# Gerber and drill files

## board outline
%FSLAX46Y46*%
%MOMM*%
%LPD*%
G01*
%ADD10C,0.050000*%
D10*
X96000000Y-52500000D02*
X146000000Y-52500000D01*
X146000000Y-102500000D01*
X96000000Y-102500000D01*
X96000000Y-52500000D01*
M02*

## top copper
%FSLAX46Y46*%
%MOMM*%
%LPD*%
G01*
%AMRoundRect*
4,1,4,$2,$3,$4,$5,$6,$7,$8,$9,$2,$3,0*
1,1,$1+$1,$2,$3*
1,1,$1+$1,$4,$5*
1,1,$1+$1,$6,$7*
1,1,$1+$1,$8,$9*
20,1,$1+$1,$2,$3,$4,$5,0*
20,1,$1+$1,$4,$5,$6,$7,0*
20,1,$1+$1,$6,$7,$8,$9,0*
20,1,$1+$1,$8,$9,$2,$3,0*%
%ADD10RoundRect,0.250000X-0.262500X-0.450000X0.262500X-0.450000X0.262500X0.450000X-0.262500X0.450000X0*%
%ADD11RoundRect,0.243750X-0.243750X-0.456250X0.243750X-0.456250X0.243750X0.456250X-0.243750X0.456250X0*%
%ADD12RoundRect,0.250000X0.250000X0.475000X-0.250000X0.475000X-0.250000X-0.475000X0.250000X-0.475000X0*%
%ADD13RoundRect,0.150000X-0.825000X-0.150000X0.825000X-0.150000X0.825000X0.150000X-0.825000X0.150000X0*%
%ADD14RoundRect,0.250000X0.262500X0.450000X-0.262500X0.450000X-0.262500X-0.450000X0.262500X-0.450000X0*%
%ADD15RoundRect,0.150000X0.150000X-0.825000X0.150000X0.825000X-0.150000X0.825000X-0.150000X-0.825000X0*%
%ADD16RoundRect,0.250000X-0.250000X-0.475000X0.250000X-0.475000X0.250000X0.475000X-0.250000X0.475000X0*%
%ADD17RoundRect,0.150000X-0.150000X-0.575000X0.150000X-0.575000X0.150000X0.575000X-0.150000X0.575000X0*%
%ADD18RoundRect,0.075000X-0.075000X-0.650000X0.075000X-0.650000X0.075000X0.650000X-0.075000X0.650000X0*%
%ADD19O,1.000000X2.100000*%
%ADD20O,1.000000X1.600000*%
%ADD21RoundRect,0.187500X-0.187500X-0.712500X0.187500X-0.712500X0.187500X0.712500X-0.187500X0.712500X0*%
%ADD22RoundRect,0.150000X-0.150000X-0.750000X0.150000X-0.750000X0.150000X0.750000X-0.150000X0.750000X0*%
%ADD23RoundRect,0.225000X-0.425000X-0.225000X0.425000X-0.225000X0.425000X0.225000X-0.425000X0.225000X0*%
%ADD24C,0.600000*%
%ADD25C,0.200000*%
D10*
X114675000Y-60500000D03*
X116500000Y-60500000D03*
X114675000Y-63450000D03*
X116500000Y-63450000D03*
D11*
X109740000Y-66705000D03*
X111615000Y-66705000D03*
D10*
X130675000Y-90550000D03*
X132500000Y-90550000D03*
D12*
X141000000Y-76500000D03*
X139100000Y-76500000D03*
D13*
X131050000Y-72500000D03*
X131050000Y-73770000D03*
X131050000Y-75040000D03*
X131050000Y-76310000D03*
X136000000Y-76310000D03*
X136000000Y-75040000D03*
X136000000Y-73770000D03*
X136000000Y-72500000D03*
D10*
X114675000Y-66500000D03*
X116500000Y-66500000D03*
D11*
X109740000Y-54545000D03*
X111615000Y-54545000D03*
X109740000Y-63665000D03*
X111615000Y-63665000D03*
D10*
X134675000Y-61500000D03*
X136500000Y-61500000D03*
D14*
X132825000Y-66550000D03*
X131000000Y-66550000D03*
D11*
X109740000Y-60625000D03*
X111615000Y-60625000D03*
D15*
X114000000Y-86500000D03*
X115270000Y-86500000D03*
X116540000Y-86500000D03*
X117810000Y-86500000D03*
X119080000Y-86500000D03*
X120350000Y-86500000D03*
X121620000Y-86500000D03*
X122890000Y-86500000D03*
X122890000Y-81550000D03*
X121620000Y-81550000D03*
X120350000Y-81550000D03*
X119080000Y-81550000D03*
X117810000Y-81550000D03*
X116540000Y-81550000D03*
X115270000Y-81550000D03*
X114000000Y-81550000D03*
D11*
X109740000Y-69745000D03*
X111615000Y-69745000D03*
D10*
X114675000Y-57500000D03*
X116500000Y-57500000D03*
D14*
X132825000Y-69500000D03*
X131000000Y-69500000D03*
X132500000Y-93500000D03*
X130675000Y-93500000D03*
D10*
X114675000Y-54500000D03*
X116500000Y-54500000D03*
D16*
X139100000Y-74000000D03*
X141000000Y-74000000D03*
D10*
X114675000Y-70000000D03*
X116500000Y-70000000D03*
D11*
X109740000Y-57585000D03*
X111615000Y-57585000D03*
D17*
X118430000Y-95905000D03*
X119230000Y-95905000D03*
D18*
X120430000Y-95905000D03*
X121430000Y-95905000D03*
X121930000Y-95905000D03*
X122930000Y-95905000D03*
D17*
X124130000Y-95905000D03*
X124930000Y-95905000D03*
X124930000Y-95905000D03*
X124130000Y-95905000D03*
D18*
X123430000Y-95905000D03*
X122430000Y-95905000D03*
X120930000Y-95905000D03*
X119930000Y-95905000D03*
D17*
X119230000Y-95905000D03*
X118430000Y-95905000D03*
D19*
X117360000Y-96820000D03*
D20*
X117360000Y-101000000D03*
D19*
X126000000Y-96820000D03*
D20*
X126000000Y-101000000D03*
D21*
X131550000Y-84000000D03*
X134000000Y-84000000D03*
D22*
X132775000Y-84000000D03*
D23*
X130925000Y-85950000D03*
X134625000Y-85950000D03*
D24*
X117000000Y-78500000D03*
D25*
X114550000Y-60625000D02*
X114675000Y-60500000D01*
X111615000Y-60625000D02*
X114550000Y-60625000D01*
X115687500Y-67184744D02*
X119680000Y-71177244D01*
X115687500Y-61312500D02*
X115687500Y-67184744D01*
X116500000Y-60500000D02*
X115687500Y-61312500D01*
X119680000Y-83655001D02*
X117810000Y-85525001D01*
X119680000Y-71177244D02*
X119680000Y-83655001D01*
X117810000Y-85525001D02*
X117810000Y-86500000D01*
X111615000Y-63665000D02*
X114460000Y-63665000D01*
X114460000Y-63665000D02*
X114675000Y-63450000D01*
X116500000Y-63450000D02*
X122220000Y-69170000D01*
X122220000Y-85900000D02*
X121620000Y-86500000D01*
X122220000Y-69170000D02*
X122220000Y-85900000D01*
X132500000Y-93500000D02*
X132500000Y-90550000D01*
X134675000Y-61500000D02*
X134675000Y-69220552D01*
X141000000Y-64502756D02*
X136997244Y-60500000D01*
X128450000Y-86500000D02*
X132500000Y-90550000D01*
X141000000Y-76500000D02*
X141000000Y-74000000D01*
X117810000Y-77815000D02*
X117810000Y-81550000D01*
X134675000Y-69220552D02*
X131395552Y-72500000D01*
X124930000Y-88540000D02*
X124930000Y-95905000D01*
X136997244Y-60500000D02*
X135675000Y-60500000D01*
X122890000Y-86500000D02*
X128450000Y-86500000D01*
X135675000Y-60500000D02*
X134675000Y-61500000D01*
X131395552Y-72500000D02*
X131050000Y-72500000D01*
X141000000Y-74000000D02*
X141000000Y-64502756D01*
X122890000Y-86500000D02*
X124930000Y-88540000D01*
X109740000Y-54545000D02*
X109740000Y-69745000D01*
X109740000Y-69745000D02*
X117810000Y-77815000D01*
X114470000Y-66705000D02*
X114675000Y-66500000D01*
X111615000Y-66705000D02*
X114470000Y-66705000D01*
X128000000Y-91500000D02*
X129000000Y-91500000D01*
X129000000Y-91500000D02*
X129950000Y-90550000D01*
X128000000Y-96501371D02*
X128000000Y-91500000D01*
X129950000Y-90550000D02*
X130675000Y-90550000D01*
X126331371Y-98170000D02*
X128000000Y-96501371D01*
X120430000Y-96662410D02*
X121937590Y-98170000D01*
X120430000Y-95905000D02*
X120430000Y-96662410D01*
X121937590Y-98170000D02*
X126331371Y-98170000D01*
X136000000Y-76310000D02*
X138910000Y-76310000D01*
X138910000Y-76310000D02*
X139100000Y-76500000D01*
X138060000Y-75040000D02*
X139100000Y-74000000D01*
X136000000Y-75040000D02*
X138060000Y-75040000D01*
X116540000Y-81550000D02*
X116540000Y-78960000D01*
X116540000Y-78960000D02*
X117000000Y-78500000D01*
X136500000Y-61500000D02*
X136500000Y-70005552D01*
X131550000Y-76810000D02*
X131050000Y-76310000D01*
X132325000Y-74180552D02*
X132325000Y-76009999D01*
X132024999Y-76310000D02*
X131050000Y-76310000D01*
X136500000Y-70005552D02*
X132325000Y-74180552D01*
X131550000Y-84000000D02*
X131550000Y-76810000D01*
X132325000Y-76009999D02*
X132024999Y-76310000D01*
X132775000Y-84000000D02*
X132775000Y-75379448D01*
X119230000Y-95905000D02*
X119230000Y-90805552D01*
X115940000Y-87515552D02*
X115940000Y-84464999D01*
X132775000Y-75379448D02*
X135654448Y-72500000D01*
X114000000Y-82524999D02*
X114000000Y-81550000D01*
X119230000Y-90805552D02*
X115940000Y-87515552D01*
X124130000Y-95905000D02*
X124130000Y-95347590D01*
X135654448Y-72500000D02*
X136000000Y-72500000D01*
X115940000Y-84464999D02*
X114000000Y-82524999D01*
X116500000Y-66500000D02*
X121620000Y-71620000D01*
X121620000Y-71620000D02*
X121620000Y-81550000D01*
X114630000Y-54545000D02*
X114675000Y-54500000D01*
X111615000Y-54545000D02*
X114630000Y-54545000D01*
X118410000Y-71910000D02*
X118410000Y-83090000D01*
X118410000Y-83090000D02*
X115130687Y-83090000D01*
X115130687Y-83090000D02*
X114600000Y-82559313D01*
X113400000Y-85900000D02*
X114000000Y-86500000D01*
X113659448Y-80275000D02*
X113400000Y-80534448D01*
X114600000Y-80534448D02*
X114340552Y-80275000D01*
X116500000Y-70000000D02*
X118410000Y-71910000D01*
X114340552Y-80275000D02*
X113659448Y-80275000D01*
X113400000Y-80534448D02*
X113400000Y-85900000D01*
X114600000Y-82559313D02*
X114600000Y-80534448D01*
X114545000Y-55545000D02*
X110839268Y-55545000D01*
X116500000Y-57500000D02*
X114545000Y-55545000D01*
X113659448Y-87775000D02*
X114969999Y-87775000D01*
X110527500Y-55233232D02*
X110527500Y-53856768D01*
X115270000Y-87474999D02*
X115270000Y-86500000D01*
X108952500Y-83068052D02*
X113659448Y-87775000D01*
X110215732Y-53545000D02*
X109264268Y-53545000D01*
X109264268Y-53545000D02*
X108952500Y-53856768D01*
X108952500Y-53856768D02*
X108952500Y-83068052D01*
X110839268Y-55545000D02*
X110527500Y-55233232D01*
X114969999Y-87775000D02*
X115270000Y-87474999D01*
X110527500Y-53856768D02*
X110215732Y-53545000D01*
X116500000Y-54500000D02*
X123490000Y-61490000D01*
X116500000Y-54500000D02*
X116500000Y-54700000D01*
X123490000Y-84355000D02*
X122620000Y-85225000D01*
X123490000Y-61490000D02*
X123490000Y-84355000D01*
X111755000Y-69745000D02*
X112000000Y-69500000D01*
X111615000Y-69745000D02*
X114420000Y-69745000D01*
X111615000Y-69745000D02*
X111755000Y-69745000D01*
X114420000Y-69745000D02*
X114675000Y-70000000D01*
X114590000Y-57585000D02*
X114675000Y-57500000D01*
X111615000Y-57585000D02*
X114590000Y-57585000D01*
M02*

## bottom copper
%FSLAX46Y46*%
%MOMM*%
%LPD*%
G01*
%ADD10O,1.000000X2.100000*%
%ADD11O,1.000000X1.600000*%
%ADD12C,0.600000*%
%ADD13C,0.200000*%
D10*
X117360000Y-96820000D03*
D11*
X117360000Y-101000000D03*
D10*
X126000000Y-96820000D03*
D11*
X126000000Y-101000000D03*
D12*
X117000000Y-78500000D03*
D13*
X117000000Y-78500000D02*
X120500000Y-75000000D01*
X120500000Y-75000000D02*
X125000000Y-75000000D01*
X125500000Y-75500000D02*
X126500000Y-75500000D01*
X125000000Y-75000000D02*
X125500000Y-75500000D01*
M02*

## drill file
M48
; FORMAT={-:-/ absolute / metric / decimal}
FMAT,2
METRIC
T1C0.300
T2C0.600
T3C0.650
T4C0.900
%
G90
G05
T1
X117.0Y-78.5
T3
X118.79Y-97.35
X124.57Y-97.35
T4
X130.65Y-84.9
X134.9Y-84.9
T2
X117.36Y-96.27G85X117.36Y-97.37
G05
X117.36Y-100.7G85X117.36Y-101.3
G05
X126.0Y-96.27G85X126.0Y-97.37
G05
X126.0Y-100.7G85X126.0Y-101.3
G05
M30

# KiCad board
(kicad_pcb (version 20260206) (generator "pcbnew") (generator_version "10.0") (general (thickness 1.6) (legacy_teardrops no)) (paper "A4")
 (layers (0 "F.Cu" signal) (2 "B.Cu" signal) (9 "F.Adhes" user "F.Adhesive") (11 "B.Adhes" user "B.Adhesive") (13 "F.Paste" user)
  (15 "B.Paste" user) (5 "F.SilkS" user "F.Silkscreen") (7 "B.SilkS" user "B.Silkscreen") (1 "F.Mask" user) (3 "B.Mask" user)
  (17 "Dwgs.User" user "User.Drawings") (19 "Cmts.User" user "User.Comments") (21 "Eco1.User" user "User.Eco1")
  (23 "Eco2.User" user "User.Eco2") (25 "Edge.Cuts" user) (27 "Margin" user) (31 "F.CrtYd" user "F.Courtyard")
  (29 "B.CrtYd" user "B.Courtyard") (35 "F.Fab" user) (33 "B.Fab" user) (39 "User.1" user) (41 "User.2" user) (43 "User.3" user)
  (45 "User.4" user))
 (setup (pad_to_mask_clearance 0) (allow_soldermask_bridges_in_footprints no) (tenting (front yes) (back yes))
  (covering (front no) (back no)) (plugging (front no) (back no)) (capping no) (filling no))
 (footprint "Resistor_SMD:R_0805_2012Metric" (layer "F.Cu") (at 115.5875 60.5)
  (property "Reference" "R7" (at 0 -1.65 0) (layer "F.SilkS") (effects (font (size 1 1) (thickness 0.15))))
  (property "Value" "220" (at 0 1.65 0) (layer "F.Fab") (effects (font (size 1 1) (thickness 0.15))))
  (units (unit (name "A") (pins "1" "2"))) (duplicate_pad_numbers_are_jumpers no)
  (pad "1" smd roundrect (at -0.9125 0) (size 1.025 1.4) (layers "F.Cu" "F.Mask" "F.Paste") (roundrect_rratio 0.243902) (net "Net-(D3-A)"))
  (pad "2" smd roundrect (at 0.9125 0) (size 1.025 1.4) (layers "F.Cu" "F.Mask" "F.Paste") (roundrect_rratio 0.243902) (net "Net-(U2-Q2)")))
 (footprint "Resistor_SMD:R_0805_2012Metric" (layer "F.Cu") (at 115.5875 63.45)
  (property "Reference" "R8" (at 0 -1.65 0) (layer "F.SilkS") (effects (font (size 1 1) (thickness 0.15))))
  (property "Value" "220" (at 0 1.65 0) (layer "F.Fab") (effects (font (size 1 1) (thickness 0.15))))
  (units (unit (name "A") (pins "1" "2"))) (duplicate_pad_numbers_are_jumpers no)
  (pad "1" smd roundrect (at -0.9125 0) (size 1.025 1.4) (layers "F.Cu" "F.Mask" "F.Paste") (roundrect_rratio 0.243902) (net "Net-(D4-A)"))
  (pad "2" smd roundrect (at 0.9125 0) (size 1.025 1.4) (layers "F.Cu" "F.Mask" "F.Paste") (roundrect_rratio 0.243902) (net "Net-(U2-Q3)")))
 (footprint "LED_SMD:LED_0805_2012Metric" (layer "F.Cu") (at 110.6775 66.705)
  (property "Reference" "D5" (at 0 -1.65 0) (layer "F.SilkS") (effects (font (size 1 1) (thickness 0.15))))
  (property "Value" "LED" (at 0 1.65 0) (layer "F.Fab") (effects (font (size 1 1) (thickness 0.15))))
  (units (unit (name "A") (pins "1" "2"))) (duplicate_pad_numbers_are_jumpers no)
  (pad "1" smd roundrect (at -0.9375 0) (size 0.975 1.4) (layers "F.Cu" "F.Mask" "F.Paste") (roundrect_rratio 0.25) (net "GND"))
  (pad "2" smd roundrect (at 0.9375 0) (size 0.975 1.4) (layers "F.Cu" "F.Mask" "F.Paste") (roundrect_rratio 0.25) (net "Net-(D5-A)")))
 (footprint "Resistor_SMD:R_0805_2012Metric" (layer "F.Cu") (at 131.5875 90.55)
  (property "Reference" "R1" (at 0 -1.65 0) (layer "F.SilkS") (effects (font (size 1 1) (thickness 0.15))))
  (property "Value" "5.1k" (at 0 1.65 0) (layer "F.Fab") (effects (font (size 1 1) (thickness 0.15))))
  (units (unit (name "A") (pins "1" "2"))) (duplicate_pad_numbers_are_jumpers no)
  (pad "1" smd roundrect (at -0.9125 0) (size 1.025 1.4) (layers "F.Cu" "F.Mask" "F.Paste") (roundrect_rratio 0.243902) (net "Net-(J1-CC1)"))
  (pad "2" smd roundrect (at 0.9125 0) (size 1.025 1.4) (layers "F.Cu" "F.Mask" "F.Paste") (roundrect_rratio 0.243902) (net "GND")))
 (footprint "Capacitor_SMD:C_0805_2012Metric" (layer "F.Cu") (at 140.05 76.5 180)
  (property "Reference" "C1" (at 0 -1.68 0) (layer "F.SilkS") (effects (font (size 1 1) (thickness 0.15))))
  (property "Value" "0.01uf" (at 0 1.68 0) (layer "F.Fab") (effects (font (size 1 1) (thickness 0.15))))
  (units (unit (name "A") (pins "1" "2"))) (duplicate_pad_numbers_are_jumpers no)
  (pad "1" smd roundrect (at -0.95 0 180) (size 1 1.45) (layers "F.Cu" "F.Mask" "F.Paste") (roundrect_rratio 0.25) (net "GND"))
  (pad "2" smd roundrect (at 0.95 0 180) (size 1 1.45) (layers "F.Cu" "F.Mask" "F.Paste") (roundrect_rratio 0.25) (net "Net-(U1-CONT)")))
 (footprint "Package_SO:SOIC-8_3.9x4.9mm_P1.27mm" (layer "F.Cu") (at 133.525 74.405)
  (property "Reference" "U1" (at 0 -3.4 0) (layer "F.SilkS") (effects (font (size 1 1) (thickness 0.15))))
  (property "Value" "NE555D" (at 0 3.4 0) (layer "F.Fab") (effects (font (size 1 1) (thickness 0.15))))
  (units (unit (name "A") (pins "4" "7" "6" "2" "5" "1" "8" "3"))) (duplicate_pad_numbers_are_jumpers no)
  (pad "1" smd roundrect (at -2.475 -1.905) (size 1.95 0.6) (layers "F.Cu" "F.Mask" "F.Paste") (roundrect_rratio 0.25) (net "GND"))
  (pad "2" smd roundrect (at -2.475 -0.635) (size 1.95 0.6) (layers "F.Cu" "F.Mask" "F.Paste") (roundrect_rratio 0.25)
   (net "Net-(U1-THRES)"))
  (pad "3" smd roundrect (at -2.475 0.635) (size 1.95 0.6) (layers "F.Cu" "F.Mask" "F.Paste") (roundrect_rratio 0.25) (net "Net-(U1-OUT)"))
  (pad "4" smd roundrect (at -2.475 1.905) (size 1.95 0.6) (layers "F.Cu" "F.Mask" "F.Paste") (roundrect_rratio 0.25)
   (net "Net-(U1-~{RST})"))
  (pad "5" smd roundrect (at 2.475 1.905) (size 1.95 0.6) (layers "F.Cu" "F.Mask" "F.Paste") (roundrect_rratio 0.25) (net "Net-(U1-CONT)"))
  (pad "6" smd roundrect (at 2.475 0.635) (size 1.95 0.6) (layers "F.Cu" "F.Mask" "F.Paste") (roundrect_rratio 0.25) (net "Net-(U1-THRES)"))
  (pad "7" smd roundrect (at 2.475 -0.635) (size 1.95 0.6) (layers "F.Cu" "F.Mask" "F.Paste") (roundrect_rratio 0.25) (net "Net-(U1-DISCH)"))
  (pad "8" smd roundrect (at 2.475 -1.905) (size 1.95 0.6) (layers "F.Cu" "F.Mask" "F.Paste") (roundrect_rratio 0.25) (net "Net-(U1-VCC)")))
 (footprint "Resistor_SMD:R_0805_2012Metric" (layer "F.Cu") (at 115.5875 66.5)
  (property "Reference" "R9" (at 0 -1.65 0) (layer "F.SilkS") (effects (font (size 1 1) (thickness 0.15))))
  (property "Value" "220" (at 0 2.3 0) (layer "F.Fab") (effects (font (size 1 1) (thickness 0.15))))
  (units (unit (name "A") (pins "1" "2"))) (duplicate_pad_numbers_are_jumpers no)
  (pad "1" smd roundrect (at -0.9125 0) (size 1.025 1.4) (layers "F.Cu" "F.Mask" "F.Paste") (roundrect_rratio 0.243902) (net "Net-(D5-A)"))
  (pad "2" smd roundrect (at 0.9125 0) (size 1.025 1.4) (layers "F.Cu" "F.Mask" "F.Paste") (roundrect_rratio 0.243902) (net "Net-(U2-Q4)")))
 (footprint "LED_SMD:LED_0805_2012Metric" (layer "F.Cu") (at 110.6775 54.545)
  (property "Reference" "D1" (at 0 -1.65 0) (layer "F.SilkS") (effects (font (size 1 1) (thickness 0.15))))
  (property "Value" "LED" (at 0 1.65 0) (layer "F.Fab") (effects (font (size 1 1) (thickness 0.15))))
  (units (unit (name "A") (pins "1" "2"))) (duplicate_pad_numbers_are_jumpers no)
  (pad "1" smd roundrect (at -0.9375 0) (size 0.975 1.4) (layers "F.Cu" "F.Mask" "F.Paste") (roundrect_rratio 0.25) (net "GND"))
  (pad "2" smd roundrect (at 0.9375 0) (size 0.975 1.4) (layers "F.Cu" "F.Mask" "F.Paste") (roundrect_rratio 0.25) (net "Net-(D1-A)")))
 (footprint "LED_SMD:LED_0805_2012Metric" (layer "F.Cu") (at 110.6775 63.665)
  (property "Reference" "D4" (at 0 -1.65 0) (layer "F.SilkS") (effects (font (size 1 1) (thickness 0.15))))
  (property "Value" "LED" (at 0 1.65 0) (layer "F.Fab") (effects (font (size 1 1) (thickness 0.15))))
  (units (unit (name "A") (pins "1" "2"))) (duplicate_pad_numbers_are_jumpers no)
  (pad "1" smd roundrect (at -0.9375 0) (size 0.975 1.4) (layers "F.Cu" "F.Mask" "F.Paste") (roundrect_rratio 0.25) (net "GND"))
  (pad "2" smd roundrect (at 0.9375 0) (size 0.975 1.4) (layers "F.Cu" "F.Mask" "F.Paste") (roundrect_rratio 0.25) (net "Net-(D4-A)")))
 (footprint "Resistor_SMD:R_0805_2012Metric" (layer "F.Cu") (at 135.5875 61.5)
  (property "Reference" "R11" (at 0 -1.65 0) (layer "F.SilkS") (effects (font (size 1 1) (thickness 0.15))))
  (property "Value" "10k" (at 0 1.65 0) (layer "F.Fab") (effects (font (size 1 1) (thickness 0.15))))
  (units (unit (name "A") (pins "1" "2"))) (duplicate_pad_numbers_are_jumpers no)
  (pad "1" smd roundrect (at -0.9125 0) (size 1.025 1.4) (layers "F.Cu" "F.Mask" "F.Paste") (roundrect_rratio 0.243902) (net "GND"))
  (pad "2" smd roundrect (at 0.9125 0) (size 1.025 1.4) (layers "F.Cu" "F.Mask" "F.Paste") (roundrect_rratio 0.243902)
   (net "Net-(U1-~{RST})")))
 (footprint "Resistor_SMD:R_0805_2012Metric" (layer "F.Cu") (at 131.9125 66.55 180)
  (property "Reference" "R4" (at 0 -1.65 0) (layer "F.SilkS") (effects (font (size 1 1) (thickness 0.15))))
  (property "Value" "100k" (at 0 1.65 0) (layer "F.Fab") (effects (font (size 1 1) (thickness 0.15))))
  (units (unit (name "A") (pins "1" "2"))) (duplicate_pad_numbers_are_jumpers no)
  (pad "1" smd roundrect (at -0.9125 0 180) (size 1.025 1.4) (layers "F.Cu" "F.Mask" "F.Paste") (roundrect_rratio 0.243902)
   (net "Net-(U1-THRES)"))
  (pad "2" smd roundrect (at 0.9125 0 180) (size 1.025 1.4) (layers "F.Cu" "F.Mask" "F.Paste") (roundrect_rratio 0.243902)
   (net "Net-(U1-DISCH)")))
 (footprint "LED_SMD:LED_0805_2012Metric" (layer "F.Cu") (at 110.6775 60.625)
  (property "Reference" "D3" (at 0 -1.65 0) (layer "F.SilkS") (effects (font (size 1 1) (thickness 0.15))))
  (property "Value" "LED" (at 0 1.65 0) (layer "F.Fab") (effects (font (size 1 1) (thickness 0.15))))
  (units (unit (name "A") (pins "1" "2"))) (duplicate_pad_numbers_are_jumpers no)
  (pad "1" smd roundrect (at -0.9375 0) (size 0.975 1.4) (layers "F.Cu" "F.Mask" "F.Paste") (roundrect_rratio 0.25) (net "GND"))
  (pad "2" smd roundrect (at 0.9375 0) (size 0.975 1.4) (layers "F.Cu" "F.Mask" "F.Paste") (roundrect_rratio 0.25) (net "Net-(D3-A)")))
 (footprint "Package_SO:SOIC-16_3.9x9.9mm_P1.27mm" (layer "F.Cu") (at 118.445 84.025 90)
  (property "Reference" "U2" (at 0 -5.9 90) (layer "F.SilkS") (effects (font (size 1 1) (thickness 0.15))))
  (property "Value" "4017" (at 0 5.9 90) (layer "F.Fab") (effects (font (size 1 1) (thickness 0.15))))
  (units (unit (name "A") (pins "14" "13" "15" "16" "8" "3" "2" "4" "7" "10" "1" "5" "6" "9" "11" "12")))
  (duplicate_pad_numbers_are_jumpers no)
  (pad "1" smd roundrect (at -2.475 -4.445 90) (size 1.95 0.6) (layers "F.Cu" "F.Mask" "F.Paste") (roundrect_rratio 0.25)
   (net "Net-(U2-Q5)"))
  (pad "2" smd roundrect (at -2.475 -3.175 90) (size 1.95 0.6) (layers "F.Cu" "F.Mask" "F.Paste") (roundrect_rratio 0.25)
   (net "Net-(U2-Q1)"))
  (pad "3" smd roundrect (at -2.475 -1.905 90) (size 1.95 0.6) (layers "F.Cu" "F.Mask" "F.Paste") (roundrect_rratio 0.25)
   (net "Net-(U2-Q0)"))
  (pad "4" smd roundrect (at -2.475 -0.635 90) (size 1.95 0.6) (layers "F.Cu" "F.Mask" "F.Paste") (roundrect_rratio 0.25)
   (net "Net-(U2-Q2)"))
  (pad "5" smd roundrect (at -2.475 0.635 90) (size 1.95 0.6) (layers "F.Cu" "F.Mask" "F.Paste") (roundrect_rratio 0.25) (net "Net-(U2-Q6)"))
  (pad "6" smd roundrect (at -2.475 1.905 90) (size 1.95 0.6) (layers "F.Cu" "F.Mask" "F.Paste") (roundrect_rratio 0.25)
   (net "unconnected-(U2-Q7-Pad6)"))
  (pad "7" smd roundrect (at -2.475 3.175 90) (size 1.95 0.6) (layers "F.Cu" "F.Mask" "F.Paste") (roundrect_rratio 0.25) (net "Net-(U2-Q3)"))
  (pad "8" smd roundrect (at -2.475 4.445 90) (size 1.95 0.6) (layers "F.Cu" "F.Mask" "F.Paste") (roundrect_rratio 0.25) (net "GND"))
  (pad "9" smd roundrect (at 2.475 4.445 90) (size 1.95 0.6) (layers "F.Cu" "F.Mask" "F.Paste") (roundrect_rratio 0.25)
   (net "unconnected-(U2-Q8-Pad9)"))
  (pad "10" smd roundrect (at 2.475 3.175 90) (size 1.95 0.6) (layers "F.Cu" "F.Mask" "F.Paste") (roundrect_rratio 0.25) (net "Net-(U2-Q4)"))
  (pad "11" smd roundrect (at 2.475 1.905 90) (size 1.95 0.6) (layers "F.Cu" "F.Mask" "F.Paste") (roundrect_rratio 0.25)
   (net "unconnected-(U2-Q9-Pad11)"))
  (pad "12" smd roundrect (at 2.475 0.635 90) (size 1.95 0.6) (layers "F.Cu" "F.Mask" "F.Paste") (roundrect_rratio 0.25)
   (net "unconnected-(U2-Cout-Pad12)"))
  (pad "13" smd roundrect (at 2.475 -0.635 90) (size 1.95 0.6) (layers "F.Cu" "F.Mask" "F.Paste") (roundrect_rratio 0.25) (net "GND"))
  (pad "14" smd roundrect (at 2.475 -1.905 90) (size 1.95 0.6) (layers "F.Cu" "F.Mask" "F.Paste") (roundrect_rratio 0.25)
   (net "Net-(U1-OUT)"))
  (pad "15" smd roundrect (at 2.475 -3.175 90) (size 1.95 0.6) (layers "F.Cu" "F.Mask" "F.Paste") (roundrect_rratio 0.25)
   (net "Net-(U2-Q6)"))
  (pad "16" smd roundrect (at 2.475 -4.445 90) (size 1.95 0.6) (layers "F.Cu" "F.Mask" "F.Paste") (roundrect_rratio 0.25)
   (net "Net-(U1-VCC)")))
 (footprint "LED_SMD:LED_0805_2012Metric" (layer "F.Cu") (at 110.6775 69.745)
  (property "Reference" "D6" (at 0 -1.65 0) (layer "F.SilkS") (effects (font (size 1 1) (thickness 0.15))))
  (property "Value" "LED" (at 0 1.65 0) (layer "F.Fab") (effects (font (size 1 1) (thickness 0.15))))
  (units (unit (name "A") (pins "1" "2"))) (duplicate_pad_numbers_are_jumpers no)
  (pad "1" smd roundrect (at -0.9375 0) (size 0.975 1.4) (layers "F.Cu" "F.Mask" "F.Paste") (roundrect_rratio 0.25) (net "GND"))
  (pad "2" smd roundrect (at 0.9375 0) (size 0.975 1.4) (layers "F.Cu" "F.Mask" "F.Paste") (roundrect_rratio 0.25) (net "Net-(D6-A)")))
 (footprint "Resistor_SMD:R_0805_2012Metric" (layer "F.Cu") (at 115.5875 57.5)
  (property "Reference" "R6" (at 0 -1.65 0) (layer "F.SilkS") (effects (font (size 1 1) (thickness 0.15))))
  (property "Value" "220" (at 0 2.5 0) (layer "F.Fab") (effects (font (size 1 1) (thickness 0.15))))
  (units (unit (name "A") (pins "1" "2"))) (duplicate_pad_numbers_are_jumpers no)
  (pad "1" smd roundrect (at -0.9125 0) (size 1.025 1.4) (layers "F.Cu" "F.Mask" "F.Paste") (roundrect_rratio 0.243902) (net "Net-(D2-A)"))
  (pad "2" smd roundrect (at 0.9125 0) (size 1.025 1.4) (layers "F.Cu" "F.Mask" "F.Paste") (roundrect_rratio 0.243902) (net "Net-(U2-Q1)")))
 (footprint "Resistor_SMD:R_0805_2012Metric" (layer "F.Cu") (at 131.9125 69.5 180)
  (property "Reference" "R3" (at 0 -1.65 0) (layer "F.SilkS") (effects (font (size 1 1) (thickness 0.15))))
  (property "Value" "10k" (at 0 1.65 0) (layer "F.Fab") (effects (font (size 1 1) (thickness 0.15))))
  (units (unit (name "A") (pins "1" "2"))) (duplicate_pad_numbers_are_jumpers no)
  (pad "1" smd roundrect (at -0.9125 0 180) (size 1.025 1.4) (layers "F.Cu" "F.Mask" "F.Paste") (roundrect_rratio 0.243902)
   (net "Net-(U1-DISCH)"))
  (pad "2" smd roundrect (at 0.9125 0 180) (size 1.025 1.4) (layers "F.Cu" "F.Mask" "F.Paste") (roundrect_rratio 0.243902)
   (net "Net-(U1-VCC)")))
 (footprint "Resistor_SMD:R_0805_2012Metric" (layer "F.Cu") (at 131.5875 93.5 180)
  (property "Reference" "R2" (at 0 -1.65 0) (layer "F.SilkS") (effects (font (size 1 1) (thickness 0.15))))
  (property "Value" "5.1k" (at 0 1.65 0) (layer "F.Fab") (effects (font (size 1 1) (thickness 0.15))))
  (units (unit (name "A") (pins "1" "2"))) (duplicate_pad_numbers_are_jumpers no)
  (pad "1" smd roundrect (at -0.9125 0 180) (size 1.025 1.4) (layers "F.Cu" "F.Mask" "F.Paste") (roundrect_rratio 0.243902) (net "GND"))
  (pad "2" smd roundrect (at 0.9125 0 180) (size 1.025 1.4) (layers "F.Cu" "F.Mask" "F.Paste") (roundrect_rratio 0.243902)
   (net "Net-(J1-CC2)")))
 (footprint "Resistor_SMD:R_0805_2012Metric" (layer "F.Cu") (at 115.5875 54.5)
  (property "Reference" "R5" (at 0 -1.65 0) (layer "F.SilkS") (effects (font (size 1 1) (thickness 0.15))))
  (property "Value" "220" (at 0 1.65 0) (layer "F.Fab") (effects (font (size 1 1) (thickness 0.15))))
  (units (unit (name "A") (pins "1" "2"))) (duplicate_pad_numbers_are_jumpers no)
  (pad "1" smd roundrect (at -0.9125 0) (size 1.025 1.4) (layers "F.Cu" "F.Mask" "F.Paste") (roundrect_rratio 0.243902) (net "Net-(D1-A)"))
  (pad "2" smd roundrect (at 0.9125 0) (size 1.025 1.4) (layers "F.Cu" "F.Mask" "F.Paste") (roundrect_rratio 0.243902) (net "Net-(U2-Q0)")))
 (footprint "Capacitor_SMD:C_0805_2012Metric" (layer "F.Cu") (at 140.05 74)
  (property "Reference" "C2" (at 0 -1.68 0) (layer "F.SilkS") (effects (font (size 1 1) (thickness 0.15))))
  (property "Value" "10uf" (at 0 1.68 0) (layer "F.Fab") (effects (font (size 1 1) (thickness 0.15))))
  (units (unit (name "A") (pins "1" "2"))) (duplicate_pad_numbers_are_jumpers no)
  (pad "1" smd roundrect (at -0.95 0) (size 1 1.45) (layers "F.Cu" "F.Mask" "F.Paste") (roundrect_rratio 0.25) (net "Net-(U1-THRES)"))
  (pad "2" smd roundrect (at 0.95 0) (size 1 1.45) (layers "F.Cu" "F.Mask" "F.Paste") (roundrect_rratio 0.25) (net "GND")))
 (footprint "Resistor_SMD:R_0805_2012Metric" (layer "F.Cu") (at 115.5875 70)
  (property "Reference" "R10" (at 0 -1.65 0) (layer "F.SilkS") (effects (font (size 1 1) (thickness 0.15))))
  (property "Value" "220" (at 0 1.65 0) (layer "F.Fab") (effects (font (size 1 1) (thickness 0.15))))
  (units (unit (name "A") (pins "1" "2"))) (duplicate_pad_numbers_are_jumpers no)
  (pad "1" smd roundrect (at -0.9125 0) (size 1.025 1.4) (layers "F.Cu" "F.Mask" "F.Paste") (roundrect_rratio 0.243902) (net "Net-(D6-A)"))
  (pad "2" smd roundrect (at 0.9125 0) (size 1.025 1.4) (layers "F.Cu" "F.Mask" "F.Paste") (roundrect_rratio 0.243902) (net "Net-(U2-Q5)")))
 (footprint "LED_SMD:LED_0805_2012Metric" (layer "F.Cu") (at 110.6775 57.585)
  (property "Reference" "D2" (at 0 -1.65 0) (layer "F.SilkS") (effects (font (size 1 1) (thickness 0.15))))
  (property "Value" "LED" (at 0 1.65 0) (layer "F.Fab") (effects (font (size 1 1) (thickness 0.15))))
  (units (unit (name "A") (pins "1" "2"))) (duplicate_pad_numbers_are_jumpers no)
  (pad "1" smd roundrect (at -0.9375 0) (size 0.975 1.4) (layers "F.Cu" "F.Mask" "F.Paste") (roundrect_rratio 0.25) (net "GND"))
  (pad "2" smd roundrect (at 0.9375 0) (size 0.975 1.4) (layers "F.Cu" "F.Mask" "F.Paste") (roundrect_rratio 0.25) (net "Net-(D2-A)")))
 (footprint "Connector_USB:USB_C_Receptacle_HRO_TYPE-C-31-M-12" (layer "F.Cu") (at 121.68 99.95)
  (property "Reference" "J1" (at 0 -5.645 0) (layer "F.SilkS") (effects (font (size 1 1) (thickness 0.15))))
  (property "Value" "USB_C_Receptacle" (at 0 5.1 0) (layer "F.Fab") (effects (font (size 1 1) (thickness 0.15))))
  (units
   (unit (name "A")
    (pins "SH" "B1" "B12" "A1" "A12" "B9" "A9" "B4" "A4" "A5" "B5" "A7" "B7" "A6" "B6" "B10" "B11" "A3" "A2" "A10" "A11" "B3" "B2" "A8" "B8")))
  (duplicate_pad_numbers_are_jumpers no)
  (pad "" np_thru_hole circle (at -2.89 -2.6) (size 0.65 0.65) (drill 0.65) (layers "*.Cu" "*.Mask"))
  (pad "" np_thru_hole circle (at 2.89 -2.6) (size 0.65 0.65) (drill 0.65) (layers "*.Cu" "*.Mask"))
  (pad "A1" smd roundrect (at -3.25 -4.045) (size 0.6 1.45) (layers "F.Cu" "F.Mask" "F.Paste") (roundrect_rratio 0.25) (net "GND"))
  (pad "A4" smd roundrect (at -2.45 -4.045) (size 0.6 1.45) (layers "F.Cu" "F.Mask" "F.Paste") (roundrect_rratio 0.25) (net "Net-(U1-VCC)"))
  (pad "A5" smd roundrect (at -1.25 -4.045) (size 0.3 1.45) (layers "F.Cu" "F.Mask" "F.Paste") (roundrect_rratio 0.25) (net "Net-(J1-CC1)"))
  (pad "A6" smd roundrect (at -0.25 -4.045) (size 0.3 1.45) (layers "F.Cu" "F.Mask" "F.Paste") (roundrect_rratio 0.25)
   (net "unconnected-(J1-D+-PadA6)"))
  (pad "A7" smd roundrect (at 0.25 -4.045) (size 0.3 1.45) (layers "F.Cu" "F.Mask" "F.Paste") (roundrect_rratio 0.25)
   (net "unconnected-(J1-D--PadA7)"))
  (pad "A8" smd roundrect (at 1.25 -4.045) (size 0.3 1.45) (layers "F.Cu" "F.Mask" "F.Paste") (roundrect_rratio 0.25)
   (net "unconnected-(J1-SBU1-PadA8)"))
  (pad "A9" smd roundrect (at 2.45 -4.045) (size 0.6 1.45) (layers "F.Cu" "F.Mask" "F.Paste") (roundrect_rratio 0.25) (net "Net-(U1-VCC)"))
  (pad "A12" smd roundrect (at 3.25 -4.045) (size 0.6 1.45) (layers "F.Cu" "F.Mask" "F.Paste") (roundrect_rratio 0.25) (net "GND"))
  (pad "B1" smd roundrect (at 3.25 -4.045) (size 0.6 1.45) (layers "F.Cu" "F.Mask" "F.Paste") (roundrect_rratio 0.25) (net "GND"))
  (pad "B4" smd roundrect (at 2.45 -4.045) (size 0.6 1.45) (layers "F.Cu" "F.Mask" "F.Paste") (roundrect_rratio 0.25) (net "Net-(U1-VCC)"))
  (pad "B5" smd roundrect (at 1.75 -4.045) (size 0.3 1.45) (layers "F.Cu" "F.Mask" "F.Paste") (roundrect_rratio 0.25) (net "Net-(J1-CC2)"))
  (pad "B6" smd roundrect (at 0.75 -4.045) (size 0.3 1.45) (layers "F.Cu" "F.Mask" "F.Paste") (roundrect_rratio 0.25)
   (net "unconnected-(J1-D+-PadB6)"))
  (pad "B7" smd roundrect (at -0.75 -4.045) (size 0.3 1.45) (layers "F.Cu" "F.Mask" "F.Paste") (roundrect_rratio 0.25)
   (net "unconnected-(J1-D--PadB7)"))
  (pad "B8" smd roundrect (at -1.75 -4.045) (size 0.3 1.45) (layers "F.Cu" "F.Mask" "F.Paste") (roundrect_rratio 0.25)
   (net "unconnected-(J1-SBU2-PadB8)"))
  (pad "B9" smd roundrect (at -2.45 -4.045) (size 0.6 1.45) (layers "F.Cu" "F.Mask" "F.Paste") (roundrect_rratio 0.25) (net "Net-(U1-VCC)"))
  (pad "B12" smd roundrect (at -3.25 -4.045) (size 0.6 1.45) (layers "F.Cu" "F.Mask" "F.Paste") (roundrect_rratio 0.25) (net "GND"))
  (pad "SH" thru_hole oval (at -4.32 -3.13) (size 1 2.1) (drill oval 0.6 1.7) (layers "*.Cu" "*.Mask") (remove_unused_layers no)
   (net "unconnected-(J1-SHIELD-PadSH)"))
  (pad "SH" thru_hole oval (at -4.32 1.05) (size 1 1.6) (drill oval 0.6 1.2) (layers "*.Cu" "*.Mask") (remove_unused_layers no)
   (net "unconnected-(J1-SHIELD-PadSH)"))
  (pad "SH" thru_hole oval (at 4.32 -3.13) (size 1 2.1) (drill oval 0.6 1.7) (layers "*.Cu" "*.Mask") (remove_unused_layers no)
   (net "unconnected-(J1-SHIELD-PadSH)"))
  (pad "SH" thru_hole oval (at 4.32 1.05) (size 1 1.6) (drill oval 0.6 1.2) (layers "*.Cu" "*.Mask") (remove_unused_layers no)
   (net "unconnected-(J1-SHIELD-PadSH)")))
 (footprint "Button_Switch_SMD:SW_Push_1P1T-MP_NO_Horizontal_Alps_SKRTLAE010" (layer "F.Cu") (at 132.775 84.9)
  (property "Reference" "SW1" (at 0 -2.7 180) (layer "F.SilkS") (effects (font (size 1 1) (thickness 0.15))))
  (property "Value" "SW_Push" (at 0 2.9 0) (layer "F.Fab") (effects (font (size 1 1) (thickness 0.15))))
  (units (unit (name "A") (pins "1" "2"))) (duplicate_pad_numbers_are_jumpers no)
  (pad "" np_thru_hole circle (at -2.125 0) (size 0.9 0.9) (drill 0.9) (layers "*.Cu" "*.Mask"))
  (pad "" np_thru_hole circle (at 2.125 0) (size 0.9 0.9) (drill 0.9) (layers "*.Cu" "*.Mask"))
  (pad "1" smd roundrect (at -1.225 -0.9) (size 0.75 1.8) (layers "F.Cu" "F.Mask" "F.Paste") (roundrect_rratio 0.25) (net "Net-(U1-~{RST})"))
  (pad "1" smd roundrect (at 1.225 -0.9) (size 0.75 1.8) (layers "F.Cu" "F.Mask" "F.Paste") (roundrect_rratio 0.25) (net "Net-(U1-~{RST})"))
  (pad "2" smd roundrect (at 0 -0.9) (size 0.6 1.8) (layers "F.Cu" "F.Mask" "F.Paste") (roundrect_rratio 0.25) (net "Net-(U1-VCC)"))
  (pad "MP" smd roundrect (at -1.85 1.05) (size 1.3 0.9) (layers "F.Cu" "F.Mask" "F.Paste") (roundrect_rratio 0.25))
  (pad "MP" smd roundrect (at 1.85 1.05) (size 1.3 0.9) (layers "F.Cu" "F.Mask" "F.Paste") (roundrect_rratio 0.25)))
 (gr_rect (start 96 52.5) (end 146 102.5) (stroke (width 0.05) (type solid)) (fill no) (layer "Edge.Cuts"))
 (segment (start 114.55 60.625) (end 114.675 60.5) (width 0.2) (layer "F.Cu") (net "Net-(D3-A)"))
 (segment (start 111.615 60.625) (end 114.55 60.625) (width 0.2) (layer "F.Cu") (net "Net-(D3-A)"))
 (segment (start 115.6875 67.184744) (end 119.68 71.177244) (width 0.2) (layer "F.Cu") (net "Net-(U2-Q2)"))
 (segment (start 115.6875 61.3125) (end 115.6875 67.184744) (width 0.2) (layer "F.Cu") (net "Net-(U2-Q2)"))
 (segment (start 116.5 60.5) (end 115.6875 61.3125) (width 0.2) (layer "F.Cu") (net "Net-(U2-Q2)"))
 (segment (start 119.68 83.655001) (end 117.81 85.525001) (width 0.2) (layer "F.Cu") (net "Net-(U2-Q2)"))
 (segment (start 119.68 71.177244) (end 119.68 83.655001) (width 0.2) (layer "F.Cu") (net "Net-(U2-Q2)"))
 (segment (start 117.81 85.525001) (end 117.81 86.5) (width 0.2) (layer "F.Cu") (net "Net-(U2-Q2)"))
 (segment (start 111.615 63.665) (end 114.46 63.665) (width 0.2) (layer "F.Cu") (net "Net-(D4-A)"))
 (segment (start 114.46 63.665) (end 114.675 63.45) (width 0.2) (layer "F.Cu") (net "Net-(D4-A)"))
 (segment (start 116.5 63.45) (end 122.22 69.17) (width 0.2) (layer "F.Cu") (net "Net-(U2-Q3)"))
 (segment (start 122.22 85.9) (end 121.62 86.5) (width 0.2) (layer "F.Cu") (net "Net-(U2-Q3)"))
 (segment (start 122.22 69.17) (end 122.22 85.9) (width 0.2) (layer "F.Cu") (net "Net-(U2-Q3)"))
 (segment (start 132.5 93.5) (end 132.5 90.55) (width 0.2) (layer "F.Cu") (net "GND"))
 (segment (start 134.675 61.5) (end 134.675 69.220552) (width 0.2) (layer "F.Cu") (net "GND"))
 (segment (start 141 64.502756) (end 136.997244 60.5) (width 0.2) (layer "F.Cu") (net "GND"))
 (segment (start 128.45 86.5) (end 132.5 90.55) (width 0.2) (layer "F.Cu") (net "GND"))
 (segment (start 141 76.5) (end 141 74) (width 0.2) (layer "F.Cu") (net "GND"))
 (segment (start 117.81 77.815) (end 117.81 81.55) (width 0.2) (layer "F.Cu") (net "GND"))
 (segment (start 134.675 69.220552) (end 131.395552 72.5) (width 0.2) (layer "F.Cu") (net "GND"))
 (segment (start 124.93 88.54) (end 124.93 95.905) (width 0.2) (layer "F.Cu") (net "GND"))
 (segment (start 136.997244 60.5) (end 135.675 60.5) (width 0.2) (layer "F.Cu") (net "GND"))
 (segment (start 122.89 86.5) (end 128.45 86.5) (width 0.2) (layer "F.Cu") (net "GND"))
 (segment (start 135.675 60.5) (end 134.675 61.5) (width 0.2) (layer "F.Cu") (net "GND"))
 (segment (start 131.395552 72.5) (end 131.05 72.5) (width 0.2) (layer "F.Cu") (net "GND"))
 (segment (start 141 74) (end 141 64.502756) (width 0.2) (layer "F.Cu") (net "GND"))
 (segment (start 122.89 86.5) (end 124.93 88.54) (width 0.2) (layer "F.Cu") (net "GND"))
 (segment (start 109.74 54.545) (end 109.74 69.745) (width 0.2) (layer "F.Cu") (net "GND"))
 (segment (start 109.74 69.745) (end 117.81 77.815) (width 0.2) (layer "F.Cu") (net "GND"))
 (segment (start 114.47 66.705) (end 114.675 66.5) (width 0.2) (layer "F.Cu") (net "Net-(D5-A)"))
 (segment (start 111.615 66.705) (end 114.47 66.705) (width 0.2) (layer "F.Cu") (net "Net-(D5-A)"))
 (segment (start 128 91.5) (end 129 91.5) (width 0.2) (layer "F.Cu") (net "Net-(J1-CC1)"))
 (segment (start 129 91.5) (end 129.95 90.55) (width 0.2) (layer "F.Cu") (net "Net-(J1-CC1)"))
 (segment (start 128 96.501371) (end 128 91.5) (width 0.2) (layer "F.Cu") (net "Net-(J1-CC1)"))
 (segment (start 129.95 90.55) (end 130.675 90.55) (width 0.2) (layer "F.Cu") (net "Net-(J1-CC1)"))
 (segment (start 126.331371 98.17) (end 128 96.501371) (width 0.2) (layer "F.Cu") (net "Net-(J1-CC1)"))
 (segment (start 120.43 96.66241) (end 121.93759 98.17) (width 0.2) (layer "F.Cu") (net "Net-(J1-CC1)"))
 (segment (start 120.43 95.905) (end 120.43 96.66241) (width 0.2) (layer "F.Cu") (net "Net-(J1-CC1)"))
 (segment (start 121.93759 98.17) (end 126.331371 98.17) (width 0.2) (layer "F.Cu") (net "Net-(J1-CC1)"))
 (segment (start 136 76.31) (end 138.91 76.31) (width 0.2) (layer "F.Cu") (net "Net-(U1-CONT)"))
 (segment (start 138.91 76.31) (end 139.1 76.5) (width 0.2) (layer "F.Cu") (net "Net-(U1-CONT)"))
 (segment (start 138.06 75.04) (end 139.1 74) (width 0.2) (layer "F.Cu") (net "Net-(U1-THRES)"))
 (segment (start 136 75.04) (end 138.06 75.04) (width 0.2) (layer "F.Cu") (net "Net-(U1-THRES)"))
 (segment (start 116.54 81.55) (end 116.54 78.96) (width 0.2) (layer "F.Cu") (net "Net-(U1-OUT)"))
 (segment (start 116.54 78.96) (end 117 78.5) (width 0.2) (layer "F.Cu") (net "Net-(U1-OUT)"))
 (via (at 117 78.5) (size 0.6) (drill 0.3) (layers "F.Cu" "B.Cu") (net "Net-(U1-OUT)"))
 (segment (start 117 78.5) (end 120.5 75) (width 0.2) (layer "B.Cu") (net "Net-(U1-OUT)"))
 (segment (start 120.5 75) (end 125 75) (width 0.2) (layer "B.Cu") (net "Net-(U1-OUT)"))
 (segment (start 125.5 75.5) (end 126.5 75.5) (width 0.2) (layer "B.Cu") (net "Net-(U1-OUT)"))
 (segment (start 125 75) (end 125.5 75.5) (width 0.2) (layer "B.Cu") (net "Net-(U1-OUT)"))
 (segment (start 136.5 61.5) (end 136.5 70.005552) (width 0.2) (layer "F.Cu") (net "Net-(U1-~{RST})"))
 (segment (start 131.55 76.81) (end 131.05 76.31) (width 0.2) (layer "F.Cu") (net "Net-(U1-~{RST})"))
 (segment (start 132.325 74.180552) (end 132.325 76.009999) (width 0.2) (layer "F.Cu") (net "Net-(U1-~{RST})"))
 (segment (start 132.024999 76.31) (end 131.05 76.31) (width 0.2) (layer "F.Cu") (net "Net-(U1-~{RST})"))
 (segment (start 136.5 70.005552) (end 132.325 74.180552) (width 0.2) (layer "F.Cu") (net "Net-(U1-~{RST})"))
 (segment (start 131.55 84) (end 131.55 76.81) (width 0.2) (layer "F.Cu") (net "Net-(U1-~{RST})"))
 (segment (start 132.325 76.009999) (end 132.024999 76.31) (width 0.2) (layer "F.Cu") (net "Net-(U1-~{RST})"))
 (segment (start 132.775 84) (end 132.775 75.379448) (width 0.2) (layer "F.Cu") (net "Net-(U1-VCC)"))
 (segment (start 119.23 95.905) (end 119.23 90.805552) (width 0.2) (layer "F.Cu") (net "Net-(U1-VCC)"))
 (segment (start 115.94 87.515552) (end 115.94 84.464999) (width 0.2) (layer "F.Cu") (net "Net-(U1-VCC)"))
 (segment (start 132.775 75.379448) (end 135.654448 72.5) (width 0.2) (layer "F.Cu") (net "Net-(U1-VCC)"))
 (segment (start 114 82.524999) (end 114 81.55) (width 0.2) (layer "F.Cu") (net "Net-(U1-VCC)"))
 (segment (start 119.23 90.805552) (end 115.94 87.515552) (width 0.2) (layer "F.Cu") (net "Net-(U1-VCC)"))
 (segment (start 124.13 95.905) (end 124.13 95.34759) (width 0.2) (layer "F.Cu") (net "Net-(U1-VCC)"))
 (segment (start 135.654448 72.5) (end 136 72.5) (width 0.2) (layer "F.Cu") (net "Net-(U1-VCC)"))
 (segment (start 115.94 84.464999) (end 114 82.524999) (width 0.2) (layer "F.Cu") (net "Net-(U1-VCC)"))
 (segment (start 116.5 66.5) (end 121.62 71.62) (width 0.2) (layer "F.Cu") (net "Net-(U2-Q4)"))
 (segment (start 121.62 71.62) (end 121.62 81.55) (width 0.2) (layer "F.Cu") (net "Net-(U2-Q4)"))
 (segment (start 114.63 54.545) (end 114.675 54.5) (width 0.2) (layer "F.Cu") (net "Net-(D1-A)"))
 (segment (start 111.615 54.545) (end 114.63 54.545) (width 0.2) (layer "F.Cu") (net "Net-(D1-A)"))
 (segment (start 118.41 71.91) (end 118.41 83.09) (width 0.2) (layer "F.Cu") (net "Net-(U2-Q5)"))
 (segment (start 118.41 83.09) (end 115.130687 83.09) (width 0.2) (layer "F.Cu") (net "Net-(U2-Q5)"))
 (segment (start 115.130687 83.09) (end 114.6 82.559313) (width 0.2) (layer "F.Cu") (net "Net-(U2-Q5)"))
 (segment (start 113.4 85.9) (end 114 86.5) (width 0.2) (layer "F.Cu") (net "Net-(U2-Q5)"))
 (segment (start 113.659448 80.275) (end 113.4 80.534448) (width 0.2) (layer "F.Cu") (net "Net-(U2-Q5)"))
 (segment (start 114.6 80.534448) (end 114.340552 80.275) (width 0.2) (layer "F.Cu") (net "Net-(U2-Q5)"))
 (segment (start 116.5 70) (end 118.41 71.91) (width 0.2) (layer "F.Cu") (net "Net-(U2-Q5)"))
 (segment (start 114.340552 80.275) (end 113.659448 80.275) (width 0.2) (layer "F.Cu") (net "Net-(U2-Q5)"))
 (segment (start 113.4 80.534448) (end 113.4 85.9) (width 0.2) (layer "F.Cu") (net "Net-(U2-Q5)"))
 (segment (start 114.6 82.559313) (end 114.6 80.534448) (width 0.2) (layer "F.Cu") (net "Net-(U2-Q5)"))
 (segment (start 114.545 55.545) (end 110.839268 55.545) (width 0.2) (layer "F.Cu") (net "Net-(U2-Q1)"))
 (segment (start 116.5 57.5) (end 114.545 55.545) (width 0.2) (layer "F.Cu") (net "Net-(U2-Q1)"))
 (segment (start 113.659448 87.775) (end 114.969999 87.775) (width 0.2) (layer "F.Cu") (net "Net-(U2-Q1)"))
 (segment (start 110.5275 55.233232) (end 110.5275 53.856768) (width 0.2) (layer "F.Cu") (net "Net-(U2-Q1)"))
 (segment (start 115.27 87.474999) (end 115.27 86.5) (width 0.2) (layer "F.Cu") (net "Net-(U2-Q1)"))
 (segment (start 108.9525 83.068052) (end 113.659448 87.775) (width 0.2) (layer "F.Cu") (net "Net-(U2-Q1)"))
 (segment (start 110.215732 53.545) (end 109.264268 53.545) (width 0.2) (layer "F.Cu") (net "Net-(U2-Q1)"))
 (segment (start 109.264268 53.545) (end 108.9525 53.856768) (width 0.2) (layer "F.Cu") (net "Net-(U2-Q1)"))
 (segment (start 108.9525 53.856768) (end 108.9525 83.068052) (width 0.2) (layer "F.Cu") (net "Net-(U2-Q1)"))
 (segment (start 110.839268 55.545) (end 110.5275 55.233232) (width 0.2) (layer "F.Cu") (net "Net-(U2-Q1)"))
 (segment (start 114.969999 87.775) (end 115.27 87.474999) (width 0.2) (layer "F.Cu") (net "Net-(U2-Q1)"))
 (segment (start 110.5275 53.856768) (end 110.215732 53.545) (width 0.2) (layer "F.Cu") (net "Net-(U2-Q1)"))
 (segment (start 116.5 54.5) (end 123.49 61.49) (width 0.2) (layer "F.Cu") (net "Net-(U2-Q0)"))
 (segment (start 116.5 54.5) (end 116.5 54.7) (width 0.2) (layer "F.Cu") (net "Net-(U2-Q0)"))
 (segment (start 123.49 84.355) (end 122.62 85.225) (width 0.2) (layer "F.Cu") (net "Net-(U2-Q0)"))
 (segment (start 123.49 61.49) (end 123.49 84.355) (width 0.2) (layer "F.Cu") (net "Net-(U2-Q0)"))
 (segment (start 111.755 69.745) (end 112 69.5) (width 0.2) (layer "F.Cu") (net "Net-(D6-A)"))
 (segment (start 111.615 69.745) (end 114.42 69.745) (width 0.2) (layer "F.Cu") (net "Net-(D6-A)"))
 (segment (start 111.615 69.745) (end 111.755 69.745) (width 0.2) (layer "F.Cu") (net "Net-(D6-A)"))
 (segment (start 114.42 69.745) (end 114.675 70) (width 0.2) (layer "F.Cu") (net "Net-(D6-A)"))
 (segment (start 114.59 57.585) (end 114.675 57.5) (width 0.2) (layer "F.Cu") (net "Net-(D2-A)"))
 (segment (start 111.615 57.585) (end 114.59 57.585) (width 0.2) (layer "F.Cu") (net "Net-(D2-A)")))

